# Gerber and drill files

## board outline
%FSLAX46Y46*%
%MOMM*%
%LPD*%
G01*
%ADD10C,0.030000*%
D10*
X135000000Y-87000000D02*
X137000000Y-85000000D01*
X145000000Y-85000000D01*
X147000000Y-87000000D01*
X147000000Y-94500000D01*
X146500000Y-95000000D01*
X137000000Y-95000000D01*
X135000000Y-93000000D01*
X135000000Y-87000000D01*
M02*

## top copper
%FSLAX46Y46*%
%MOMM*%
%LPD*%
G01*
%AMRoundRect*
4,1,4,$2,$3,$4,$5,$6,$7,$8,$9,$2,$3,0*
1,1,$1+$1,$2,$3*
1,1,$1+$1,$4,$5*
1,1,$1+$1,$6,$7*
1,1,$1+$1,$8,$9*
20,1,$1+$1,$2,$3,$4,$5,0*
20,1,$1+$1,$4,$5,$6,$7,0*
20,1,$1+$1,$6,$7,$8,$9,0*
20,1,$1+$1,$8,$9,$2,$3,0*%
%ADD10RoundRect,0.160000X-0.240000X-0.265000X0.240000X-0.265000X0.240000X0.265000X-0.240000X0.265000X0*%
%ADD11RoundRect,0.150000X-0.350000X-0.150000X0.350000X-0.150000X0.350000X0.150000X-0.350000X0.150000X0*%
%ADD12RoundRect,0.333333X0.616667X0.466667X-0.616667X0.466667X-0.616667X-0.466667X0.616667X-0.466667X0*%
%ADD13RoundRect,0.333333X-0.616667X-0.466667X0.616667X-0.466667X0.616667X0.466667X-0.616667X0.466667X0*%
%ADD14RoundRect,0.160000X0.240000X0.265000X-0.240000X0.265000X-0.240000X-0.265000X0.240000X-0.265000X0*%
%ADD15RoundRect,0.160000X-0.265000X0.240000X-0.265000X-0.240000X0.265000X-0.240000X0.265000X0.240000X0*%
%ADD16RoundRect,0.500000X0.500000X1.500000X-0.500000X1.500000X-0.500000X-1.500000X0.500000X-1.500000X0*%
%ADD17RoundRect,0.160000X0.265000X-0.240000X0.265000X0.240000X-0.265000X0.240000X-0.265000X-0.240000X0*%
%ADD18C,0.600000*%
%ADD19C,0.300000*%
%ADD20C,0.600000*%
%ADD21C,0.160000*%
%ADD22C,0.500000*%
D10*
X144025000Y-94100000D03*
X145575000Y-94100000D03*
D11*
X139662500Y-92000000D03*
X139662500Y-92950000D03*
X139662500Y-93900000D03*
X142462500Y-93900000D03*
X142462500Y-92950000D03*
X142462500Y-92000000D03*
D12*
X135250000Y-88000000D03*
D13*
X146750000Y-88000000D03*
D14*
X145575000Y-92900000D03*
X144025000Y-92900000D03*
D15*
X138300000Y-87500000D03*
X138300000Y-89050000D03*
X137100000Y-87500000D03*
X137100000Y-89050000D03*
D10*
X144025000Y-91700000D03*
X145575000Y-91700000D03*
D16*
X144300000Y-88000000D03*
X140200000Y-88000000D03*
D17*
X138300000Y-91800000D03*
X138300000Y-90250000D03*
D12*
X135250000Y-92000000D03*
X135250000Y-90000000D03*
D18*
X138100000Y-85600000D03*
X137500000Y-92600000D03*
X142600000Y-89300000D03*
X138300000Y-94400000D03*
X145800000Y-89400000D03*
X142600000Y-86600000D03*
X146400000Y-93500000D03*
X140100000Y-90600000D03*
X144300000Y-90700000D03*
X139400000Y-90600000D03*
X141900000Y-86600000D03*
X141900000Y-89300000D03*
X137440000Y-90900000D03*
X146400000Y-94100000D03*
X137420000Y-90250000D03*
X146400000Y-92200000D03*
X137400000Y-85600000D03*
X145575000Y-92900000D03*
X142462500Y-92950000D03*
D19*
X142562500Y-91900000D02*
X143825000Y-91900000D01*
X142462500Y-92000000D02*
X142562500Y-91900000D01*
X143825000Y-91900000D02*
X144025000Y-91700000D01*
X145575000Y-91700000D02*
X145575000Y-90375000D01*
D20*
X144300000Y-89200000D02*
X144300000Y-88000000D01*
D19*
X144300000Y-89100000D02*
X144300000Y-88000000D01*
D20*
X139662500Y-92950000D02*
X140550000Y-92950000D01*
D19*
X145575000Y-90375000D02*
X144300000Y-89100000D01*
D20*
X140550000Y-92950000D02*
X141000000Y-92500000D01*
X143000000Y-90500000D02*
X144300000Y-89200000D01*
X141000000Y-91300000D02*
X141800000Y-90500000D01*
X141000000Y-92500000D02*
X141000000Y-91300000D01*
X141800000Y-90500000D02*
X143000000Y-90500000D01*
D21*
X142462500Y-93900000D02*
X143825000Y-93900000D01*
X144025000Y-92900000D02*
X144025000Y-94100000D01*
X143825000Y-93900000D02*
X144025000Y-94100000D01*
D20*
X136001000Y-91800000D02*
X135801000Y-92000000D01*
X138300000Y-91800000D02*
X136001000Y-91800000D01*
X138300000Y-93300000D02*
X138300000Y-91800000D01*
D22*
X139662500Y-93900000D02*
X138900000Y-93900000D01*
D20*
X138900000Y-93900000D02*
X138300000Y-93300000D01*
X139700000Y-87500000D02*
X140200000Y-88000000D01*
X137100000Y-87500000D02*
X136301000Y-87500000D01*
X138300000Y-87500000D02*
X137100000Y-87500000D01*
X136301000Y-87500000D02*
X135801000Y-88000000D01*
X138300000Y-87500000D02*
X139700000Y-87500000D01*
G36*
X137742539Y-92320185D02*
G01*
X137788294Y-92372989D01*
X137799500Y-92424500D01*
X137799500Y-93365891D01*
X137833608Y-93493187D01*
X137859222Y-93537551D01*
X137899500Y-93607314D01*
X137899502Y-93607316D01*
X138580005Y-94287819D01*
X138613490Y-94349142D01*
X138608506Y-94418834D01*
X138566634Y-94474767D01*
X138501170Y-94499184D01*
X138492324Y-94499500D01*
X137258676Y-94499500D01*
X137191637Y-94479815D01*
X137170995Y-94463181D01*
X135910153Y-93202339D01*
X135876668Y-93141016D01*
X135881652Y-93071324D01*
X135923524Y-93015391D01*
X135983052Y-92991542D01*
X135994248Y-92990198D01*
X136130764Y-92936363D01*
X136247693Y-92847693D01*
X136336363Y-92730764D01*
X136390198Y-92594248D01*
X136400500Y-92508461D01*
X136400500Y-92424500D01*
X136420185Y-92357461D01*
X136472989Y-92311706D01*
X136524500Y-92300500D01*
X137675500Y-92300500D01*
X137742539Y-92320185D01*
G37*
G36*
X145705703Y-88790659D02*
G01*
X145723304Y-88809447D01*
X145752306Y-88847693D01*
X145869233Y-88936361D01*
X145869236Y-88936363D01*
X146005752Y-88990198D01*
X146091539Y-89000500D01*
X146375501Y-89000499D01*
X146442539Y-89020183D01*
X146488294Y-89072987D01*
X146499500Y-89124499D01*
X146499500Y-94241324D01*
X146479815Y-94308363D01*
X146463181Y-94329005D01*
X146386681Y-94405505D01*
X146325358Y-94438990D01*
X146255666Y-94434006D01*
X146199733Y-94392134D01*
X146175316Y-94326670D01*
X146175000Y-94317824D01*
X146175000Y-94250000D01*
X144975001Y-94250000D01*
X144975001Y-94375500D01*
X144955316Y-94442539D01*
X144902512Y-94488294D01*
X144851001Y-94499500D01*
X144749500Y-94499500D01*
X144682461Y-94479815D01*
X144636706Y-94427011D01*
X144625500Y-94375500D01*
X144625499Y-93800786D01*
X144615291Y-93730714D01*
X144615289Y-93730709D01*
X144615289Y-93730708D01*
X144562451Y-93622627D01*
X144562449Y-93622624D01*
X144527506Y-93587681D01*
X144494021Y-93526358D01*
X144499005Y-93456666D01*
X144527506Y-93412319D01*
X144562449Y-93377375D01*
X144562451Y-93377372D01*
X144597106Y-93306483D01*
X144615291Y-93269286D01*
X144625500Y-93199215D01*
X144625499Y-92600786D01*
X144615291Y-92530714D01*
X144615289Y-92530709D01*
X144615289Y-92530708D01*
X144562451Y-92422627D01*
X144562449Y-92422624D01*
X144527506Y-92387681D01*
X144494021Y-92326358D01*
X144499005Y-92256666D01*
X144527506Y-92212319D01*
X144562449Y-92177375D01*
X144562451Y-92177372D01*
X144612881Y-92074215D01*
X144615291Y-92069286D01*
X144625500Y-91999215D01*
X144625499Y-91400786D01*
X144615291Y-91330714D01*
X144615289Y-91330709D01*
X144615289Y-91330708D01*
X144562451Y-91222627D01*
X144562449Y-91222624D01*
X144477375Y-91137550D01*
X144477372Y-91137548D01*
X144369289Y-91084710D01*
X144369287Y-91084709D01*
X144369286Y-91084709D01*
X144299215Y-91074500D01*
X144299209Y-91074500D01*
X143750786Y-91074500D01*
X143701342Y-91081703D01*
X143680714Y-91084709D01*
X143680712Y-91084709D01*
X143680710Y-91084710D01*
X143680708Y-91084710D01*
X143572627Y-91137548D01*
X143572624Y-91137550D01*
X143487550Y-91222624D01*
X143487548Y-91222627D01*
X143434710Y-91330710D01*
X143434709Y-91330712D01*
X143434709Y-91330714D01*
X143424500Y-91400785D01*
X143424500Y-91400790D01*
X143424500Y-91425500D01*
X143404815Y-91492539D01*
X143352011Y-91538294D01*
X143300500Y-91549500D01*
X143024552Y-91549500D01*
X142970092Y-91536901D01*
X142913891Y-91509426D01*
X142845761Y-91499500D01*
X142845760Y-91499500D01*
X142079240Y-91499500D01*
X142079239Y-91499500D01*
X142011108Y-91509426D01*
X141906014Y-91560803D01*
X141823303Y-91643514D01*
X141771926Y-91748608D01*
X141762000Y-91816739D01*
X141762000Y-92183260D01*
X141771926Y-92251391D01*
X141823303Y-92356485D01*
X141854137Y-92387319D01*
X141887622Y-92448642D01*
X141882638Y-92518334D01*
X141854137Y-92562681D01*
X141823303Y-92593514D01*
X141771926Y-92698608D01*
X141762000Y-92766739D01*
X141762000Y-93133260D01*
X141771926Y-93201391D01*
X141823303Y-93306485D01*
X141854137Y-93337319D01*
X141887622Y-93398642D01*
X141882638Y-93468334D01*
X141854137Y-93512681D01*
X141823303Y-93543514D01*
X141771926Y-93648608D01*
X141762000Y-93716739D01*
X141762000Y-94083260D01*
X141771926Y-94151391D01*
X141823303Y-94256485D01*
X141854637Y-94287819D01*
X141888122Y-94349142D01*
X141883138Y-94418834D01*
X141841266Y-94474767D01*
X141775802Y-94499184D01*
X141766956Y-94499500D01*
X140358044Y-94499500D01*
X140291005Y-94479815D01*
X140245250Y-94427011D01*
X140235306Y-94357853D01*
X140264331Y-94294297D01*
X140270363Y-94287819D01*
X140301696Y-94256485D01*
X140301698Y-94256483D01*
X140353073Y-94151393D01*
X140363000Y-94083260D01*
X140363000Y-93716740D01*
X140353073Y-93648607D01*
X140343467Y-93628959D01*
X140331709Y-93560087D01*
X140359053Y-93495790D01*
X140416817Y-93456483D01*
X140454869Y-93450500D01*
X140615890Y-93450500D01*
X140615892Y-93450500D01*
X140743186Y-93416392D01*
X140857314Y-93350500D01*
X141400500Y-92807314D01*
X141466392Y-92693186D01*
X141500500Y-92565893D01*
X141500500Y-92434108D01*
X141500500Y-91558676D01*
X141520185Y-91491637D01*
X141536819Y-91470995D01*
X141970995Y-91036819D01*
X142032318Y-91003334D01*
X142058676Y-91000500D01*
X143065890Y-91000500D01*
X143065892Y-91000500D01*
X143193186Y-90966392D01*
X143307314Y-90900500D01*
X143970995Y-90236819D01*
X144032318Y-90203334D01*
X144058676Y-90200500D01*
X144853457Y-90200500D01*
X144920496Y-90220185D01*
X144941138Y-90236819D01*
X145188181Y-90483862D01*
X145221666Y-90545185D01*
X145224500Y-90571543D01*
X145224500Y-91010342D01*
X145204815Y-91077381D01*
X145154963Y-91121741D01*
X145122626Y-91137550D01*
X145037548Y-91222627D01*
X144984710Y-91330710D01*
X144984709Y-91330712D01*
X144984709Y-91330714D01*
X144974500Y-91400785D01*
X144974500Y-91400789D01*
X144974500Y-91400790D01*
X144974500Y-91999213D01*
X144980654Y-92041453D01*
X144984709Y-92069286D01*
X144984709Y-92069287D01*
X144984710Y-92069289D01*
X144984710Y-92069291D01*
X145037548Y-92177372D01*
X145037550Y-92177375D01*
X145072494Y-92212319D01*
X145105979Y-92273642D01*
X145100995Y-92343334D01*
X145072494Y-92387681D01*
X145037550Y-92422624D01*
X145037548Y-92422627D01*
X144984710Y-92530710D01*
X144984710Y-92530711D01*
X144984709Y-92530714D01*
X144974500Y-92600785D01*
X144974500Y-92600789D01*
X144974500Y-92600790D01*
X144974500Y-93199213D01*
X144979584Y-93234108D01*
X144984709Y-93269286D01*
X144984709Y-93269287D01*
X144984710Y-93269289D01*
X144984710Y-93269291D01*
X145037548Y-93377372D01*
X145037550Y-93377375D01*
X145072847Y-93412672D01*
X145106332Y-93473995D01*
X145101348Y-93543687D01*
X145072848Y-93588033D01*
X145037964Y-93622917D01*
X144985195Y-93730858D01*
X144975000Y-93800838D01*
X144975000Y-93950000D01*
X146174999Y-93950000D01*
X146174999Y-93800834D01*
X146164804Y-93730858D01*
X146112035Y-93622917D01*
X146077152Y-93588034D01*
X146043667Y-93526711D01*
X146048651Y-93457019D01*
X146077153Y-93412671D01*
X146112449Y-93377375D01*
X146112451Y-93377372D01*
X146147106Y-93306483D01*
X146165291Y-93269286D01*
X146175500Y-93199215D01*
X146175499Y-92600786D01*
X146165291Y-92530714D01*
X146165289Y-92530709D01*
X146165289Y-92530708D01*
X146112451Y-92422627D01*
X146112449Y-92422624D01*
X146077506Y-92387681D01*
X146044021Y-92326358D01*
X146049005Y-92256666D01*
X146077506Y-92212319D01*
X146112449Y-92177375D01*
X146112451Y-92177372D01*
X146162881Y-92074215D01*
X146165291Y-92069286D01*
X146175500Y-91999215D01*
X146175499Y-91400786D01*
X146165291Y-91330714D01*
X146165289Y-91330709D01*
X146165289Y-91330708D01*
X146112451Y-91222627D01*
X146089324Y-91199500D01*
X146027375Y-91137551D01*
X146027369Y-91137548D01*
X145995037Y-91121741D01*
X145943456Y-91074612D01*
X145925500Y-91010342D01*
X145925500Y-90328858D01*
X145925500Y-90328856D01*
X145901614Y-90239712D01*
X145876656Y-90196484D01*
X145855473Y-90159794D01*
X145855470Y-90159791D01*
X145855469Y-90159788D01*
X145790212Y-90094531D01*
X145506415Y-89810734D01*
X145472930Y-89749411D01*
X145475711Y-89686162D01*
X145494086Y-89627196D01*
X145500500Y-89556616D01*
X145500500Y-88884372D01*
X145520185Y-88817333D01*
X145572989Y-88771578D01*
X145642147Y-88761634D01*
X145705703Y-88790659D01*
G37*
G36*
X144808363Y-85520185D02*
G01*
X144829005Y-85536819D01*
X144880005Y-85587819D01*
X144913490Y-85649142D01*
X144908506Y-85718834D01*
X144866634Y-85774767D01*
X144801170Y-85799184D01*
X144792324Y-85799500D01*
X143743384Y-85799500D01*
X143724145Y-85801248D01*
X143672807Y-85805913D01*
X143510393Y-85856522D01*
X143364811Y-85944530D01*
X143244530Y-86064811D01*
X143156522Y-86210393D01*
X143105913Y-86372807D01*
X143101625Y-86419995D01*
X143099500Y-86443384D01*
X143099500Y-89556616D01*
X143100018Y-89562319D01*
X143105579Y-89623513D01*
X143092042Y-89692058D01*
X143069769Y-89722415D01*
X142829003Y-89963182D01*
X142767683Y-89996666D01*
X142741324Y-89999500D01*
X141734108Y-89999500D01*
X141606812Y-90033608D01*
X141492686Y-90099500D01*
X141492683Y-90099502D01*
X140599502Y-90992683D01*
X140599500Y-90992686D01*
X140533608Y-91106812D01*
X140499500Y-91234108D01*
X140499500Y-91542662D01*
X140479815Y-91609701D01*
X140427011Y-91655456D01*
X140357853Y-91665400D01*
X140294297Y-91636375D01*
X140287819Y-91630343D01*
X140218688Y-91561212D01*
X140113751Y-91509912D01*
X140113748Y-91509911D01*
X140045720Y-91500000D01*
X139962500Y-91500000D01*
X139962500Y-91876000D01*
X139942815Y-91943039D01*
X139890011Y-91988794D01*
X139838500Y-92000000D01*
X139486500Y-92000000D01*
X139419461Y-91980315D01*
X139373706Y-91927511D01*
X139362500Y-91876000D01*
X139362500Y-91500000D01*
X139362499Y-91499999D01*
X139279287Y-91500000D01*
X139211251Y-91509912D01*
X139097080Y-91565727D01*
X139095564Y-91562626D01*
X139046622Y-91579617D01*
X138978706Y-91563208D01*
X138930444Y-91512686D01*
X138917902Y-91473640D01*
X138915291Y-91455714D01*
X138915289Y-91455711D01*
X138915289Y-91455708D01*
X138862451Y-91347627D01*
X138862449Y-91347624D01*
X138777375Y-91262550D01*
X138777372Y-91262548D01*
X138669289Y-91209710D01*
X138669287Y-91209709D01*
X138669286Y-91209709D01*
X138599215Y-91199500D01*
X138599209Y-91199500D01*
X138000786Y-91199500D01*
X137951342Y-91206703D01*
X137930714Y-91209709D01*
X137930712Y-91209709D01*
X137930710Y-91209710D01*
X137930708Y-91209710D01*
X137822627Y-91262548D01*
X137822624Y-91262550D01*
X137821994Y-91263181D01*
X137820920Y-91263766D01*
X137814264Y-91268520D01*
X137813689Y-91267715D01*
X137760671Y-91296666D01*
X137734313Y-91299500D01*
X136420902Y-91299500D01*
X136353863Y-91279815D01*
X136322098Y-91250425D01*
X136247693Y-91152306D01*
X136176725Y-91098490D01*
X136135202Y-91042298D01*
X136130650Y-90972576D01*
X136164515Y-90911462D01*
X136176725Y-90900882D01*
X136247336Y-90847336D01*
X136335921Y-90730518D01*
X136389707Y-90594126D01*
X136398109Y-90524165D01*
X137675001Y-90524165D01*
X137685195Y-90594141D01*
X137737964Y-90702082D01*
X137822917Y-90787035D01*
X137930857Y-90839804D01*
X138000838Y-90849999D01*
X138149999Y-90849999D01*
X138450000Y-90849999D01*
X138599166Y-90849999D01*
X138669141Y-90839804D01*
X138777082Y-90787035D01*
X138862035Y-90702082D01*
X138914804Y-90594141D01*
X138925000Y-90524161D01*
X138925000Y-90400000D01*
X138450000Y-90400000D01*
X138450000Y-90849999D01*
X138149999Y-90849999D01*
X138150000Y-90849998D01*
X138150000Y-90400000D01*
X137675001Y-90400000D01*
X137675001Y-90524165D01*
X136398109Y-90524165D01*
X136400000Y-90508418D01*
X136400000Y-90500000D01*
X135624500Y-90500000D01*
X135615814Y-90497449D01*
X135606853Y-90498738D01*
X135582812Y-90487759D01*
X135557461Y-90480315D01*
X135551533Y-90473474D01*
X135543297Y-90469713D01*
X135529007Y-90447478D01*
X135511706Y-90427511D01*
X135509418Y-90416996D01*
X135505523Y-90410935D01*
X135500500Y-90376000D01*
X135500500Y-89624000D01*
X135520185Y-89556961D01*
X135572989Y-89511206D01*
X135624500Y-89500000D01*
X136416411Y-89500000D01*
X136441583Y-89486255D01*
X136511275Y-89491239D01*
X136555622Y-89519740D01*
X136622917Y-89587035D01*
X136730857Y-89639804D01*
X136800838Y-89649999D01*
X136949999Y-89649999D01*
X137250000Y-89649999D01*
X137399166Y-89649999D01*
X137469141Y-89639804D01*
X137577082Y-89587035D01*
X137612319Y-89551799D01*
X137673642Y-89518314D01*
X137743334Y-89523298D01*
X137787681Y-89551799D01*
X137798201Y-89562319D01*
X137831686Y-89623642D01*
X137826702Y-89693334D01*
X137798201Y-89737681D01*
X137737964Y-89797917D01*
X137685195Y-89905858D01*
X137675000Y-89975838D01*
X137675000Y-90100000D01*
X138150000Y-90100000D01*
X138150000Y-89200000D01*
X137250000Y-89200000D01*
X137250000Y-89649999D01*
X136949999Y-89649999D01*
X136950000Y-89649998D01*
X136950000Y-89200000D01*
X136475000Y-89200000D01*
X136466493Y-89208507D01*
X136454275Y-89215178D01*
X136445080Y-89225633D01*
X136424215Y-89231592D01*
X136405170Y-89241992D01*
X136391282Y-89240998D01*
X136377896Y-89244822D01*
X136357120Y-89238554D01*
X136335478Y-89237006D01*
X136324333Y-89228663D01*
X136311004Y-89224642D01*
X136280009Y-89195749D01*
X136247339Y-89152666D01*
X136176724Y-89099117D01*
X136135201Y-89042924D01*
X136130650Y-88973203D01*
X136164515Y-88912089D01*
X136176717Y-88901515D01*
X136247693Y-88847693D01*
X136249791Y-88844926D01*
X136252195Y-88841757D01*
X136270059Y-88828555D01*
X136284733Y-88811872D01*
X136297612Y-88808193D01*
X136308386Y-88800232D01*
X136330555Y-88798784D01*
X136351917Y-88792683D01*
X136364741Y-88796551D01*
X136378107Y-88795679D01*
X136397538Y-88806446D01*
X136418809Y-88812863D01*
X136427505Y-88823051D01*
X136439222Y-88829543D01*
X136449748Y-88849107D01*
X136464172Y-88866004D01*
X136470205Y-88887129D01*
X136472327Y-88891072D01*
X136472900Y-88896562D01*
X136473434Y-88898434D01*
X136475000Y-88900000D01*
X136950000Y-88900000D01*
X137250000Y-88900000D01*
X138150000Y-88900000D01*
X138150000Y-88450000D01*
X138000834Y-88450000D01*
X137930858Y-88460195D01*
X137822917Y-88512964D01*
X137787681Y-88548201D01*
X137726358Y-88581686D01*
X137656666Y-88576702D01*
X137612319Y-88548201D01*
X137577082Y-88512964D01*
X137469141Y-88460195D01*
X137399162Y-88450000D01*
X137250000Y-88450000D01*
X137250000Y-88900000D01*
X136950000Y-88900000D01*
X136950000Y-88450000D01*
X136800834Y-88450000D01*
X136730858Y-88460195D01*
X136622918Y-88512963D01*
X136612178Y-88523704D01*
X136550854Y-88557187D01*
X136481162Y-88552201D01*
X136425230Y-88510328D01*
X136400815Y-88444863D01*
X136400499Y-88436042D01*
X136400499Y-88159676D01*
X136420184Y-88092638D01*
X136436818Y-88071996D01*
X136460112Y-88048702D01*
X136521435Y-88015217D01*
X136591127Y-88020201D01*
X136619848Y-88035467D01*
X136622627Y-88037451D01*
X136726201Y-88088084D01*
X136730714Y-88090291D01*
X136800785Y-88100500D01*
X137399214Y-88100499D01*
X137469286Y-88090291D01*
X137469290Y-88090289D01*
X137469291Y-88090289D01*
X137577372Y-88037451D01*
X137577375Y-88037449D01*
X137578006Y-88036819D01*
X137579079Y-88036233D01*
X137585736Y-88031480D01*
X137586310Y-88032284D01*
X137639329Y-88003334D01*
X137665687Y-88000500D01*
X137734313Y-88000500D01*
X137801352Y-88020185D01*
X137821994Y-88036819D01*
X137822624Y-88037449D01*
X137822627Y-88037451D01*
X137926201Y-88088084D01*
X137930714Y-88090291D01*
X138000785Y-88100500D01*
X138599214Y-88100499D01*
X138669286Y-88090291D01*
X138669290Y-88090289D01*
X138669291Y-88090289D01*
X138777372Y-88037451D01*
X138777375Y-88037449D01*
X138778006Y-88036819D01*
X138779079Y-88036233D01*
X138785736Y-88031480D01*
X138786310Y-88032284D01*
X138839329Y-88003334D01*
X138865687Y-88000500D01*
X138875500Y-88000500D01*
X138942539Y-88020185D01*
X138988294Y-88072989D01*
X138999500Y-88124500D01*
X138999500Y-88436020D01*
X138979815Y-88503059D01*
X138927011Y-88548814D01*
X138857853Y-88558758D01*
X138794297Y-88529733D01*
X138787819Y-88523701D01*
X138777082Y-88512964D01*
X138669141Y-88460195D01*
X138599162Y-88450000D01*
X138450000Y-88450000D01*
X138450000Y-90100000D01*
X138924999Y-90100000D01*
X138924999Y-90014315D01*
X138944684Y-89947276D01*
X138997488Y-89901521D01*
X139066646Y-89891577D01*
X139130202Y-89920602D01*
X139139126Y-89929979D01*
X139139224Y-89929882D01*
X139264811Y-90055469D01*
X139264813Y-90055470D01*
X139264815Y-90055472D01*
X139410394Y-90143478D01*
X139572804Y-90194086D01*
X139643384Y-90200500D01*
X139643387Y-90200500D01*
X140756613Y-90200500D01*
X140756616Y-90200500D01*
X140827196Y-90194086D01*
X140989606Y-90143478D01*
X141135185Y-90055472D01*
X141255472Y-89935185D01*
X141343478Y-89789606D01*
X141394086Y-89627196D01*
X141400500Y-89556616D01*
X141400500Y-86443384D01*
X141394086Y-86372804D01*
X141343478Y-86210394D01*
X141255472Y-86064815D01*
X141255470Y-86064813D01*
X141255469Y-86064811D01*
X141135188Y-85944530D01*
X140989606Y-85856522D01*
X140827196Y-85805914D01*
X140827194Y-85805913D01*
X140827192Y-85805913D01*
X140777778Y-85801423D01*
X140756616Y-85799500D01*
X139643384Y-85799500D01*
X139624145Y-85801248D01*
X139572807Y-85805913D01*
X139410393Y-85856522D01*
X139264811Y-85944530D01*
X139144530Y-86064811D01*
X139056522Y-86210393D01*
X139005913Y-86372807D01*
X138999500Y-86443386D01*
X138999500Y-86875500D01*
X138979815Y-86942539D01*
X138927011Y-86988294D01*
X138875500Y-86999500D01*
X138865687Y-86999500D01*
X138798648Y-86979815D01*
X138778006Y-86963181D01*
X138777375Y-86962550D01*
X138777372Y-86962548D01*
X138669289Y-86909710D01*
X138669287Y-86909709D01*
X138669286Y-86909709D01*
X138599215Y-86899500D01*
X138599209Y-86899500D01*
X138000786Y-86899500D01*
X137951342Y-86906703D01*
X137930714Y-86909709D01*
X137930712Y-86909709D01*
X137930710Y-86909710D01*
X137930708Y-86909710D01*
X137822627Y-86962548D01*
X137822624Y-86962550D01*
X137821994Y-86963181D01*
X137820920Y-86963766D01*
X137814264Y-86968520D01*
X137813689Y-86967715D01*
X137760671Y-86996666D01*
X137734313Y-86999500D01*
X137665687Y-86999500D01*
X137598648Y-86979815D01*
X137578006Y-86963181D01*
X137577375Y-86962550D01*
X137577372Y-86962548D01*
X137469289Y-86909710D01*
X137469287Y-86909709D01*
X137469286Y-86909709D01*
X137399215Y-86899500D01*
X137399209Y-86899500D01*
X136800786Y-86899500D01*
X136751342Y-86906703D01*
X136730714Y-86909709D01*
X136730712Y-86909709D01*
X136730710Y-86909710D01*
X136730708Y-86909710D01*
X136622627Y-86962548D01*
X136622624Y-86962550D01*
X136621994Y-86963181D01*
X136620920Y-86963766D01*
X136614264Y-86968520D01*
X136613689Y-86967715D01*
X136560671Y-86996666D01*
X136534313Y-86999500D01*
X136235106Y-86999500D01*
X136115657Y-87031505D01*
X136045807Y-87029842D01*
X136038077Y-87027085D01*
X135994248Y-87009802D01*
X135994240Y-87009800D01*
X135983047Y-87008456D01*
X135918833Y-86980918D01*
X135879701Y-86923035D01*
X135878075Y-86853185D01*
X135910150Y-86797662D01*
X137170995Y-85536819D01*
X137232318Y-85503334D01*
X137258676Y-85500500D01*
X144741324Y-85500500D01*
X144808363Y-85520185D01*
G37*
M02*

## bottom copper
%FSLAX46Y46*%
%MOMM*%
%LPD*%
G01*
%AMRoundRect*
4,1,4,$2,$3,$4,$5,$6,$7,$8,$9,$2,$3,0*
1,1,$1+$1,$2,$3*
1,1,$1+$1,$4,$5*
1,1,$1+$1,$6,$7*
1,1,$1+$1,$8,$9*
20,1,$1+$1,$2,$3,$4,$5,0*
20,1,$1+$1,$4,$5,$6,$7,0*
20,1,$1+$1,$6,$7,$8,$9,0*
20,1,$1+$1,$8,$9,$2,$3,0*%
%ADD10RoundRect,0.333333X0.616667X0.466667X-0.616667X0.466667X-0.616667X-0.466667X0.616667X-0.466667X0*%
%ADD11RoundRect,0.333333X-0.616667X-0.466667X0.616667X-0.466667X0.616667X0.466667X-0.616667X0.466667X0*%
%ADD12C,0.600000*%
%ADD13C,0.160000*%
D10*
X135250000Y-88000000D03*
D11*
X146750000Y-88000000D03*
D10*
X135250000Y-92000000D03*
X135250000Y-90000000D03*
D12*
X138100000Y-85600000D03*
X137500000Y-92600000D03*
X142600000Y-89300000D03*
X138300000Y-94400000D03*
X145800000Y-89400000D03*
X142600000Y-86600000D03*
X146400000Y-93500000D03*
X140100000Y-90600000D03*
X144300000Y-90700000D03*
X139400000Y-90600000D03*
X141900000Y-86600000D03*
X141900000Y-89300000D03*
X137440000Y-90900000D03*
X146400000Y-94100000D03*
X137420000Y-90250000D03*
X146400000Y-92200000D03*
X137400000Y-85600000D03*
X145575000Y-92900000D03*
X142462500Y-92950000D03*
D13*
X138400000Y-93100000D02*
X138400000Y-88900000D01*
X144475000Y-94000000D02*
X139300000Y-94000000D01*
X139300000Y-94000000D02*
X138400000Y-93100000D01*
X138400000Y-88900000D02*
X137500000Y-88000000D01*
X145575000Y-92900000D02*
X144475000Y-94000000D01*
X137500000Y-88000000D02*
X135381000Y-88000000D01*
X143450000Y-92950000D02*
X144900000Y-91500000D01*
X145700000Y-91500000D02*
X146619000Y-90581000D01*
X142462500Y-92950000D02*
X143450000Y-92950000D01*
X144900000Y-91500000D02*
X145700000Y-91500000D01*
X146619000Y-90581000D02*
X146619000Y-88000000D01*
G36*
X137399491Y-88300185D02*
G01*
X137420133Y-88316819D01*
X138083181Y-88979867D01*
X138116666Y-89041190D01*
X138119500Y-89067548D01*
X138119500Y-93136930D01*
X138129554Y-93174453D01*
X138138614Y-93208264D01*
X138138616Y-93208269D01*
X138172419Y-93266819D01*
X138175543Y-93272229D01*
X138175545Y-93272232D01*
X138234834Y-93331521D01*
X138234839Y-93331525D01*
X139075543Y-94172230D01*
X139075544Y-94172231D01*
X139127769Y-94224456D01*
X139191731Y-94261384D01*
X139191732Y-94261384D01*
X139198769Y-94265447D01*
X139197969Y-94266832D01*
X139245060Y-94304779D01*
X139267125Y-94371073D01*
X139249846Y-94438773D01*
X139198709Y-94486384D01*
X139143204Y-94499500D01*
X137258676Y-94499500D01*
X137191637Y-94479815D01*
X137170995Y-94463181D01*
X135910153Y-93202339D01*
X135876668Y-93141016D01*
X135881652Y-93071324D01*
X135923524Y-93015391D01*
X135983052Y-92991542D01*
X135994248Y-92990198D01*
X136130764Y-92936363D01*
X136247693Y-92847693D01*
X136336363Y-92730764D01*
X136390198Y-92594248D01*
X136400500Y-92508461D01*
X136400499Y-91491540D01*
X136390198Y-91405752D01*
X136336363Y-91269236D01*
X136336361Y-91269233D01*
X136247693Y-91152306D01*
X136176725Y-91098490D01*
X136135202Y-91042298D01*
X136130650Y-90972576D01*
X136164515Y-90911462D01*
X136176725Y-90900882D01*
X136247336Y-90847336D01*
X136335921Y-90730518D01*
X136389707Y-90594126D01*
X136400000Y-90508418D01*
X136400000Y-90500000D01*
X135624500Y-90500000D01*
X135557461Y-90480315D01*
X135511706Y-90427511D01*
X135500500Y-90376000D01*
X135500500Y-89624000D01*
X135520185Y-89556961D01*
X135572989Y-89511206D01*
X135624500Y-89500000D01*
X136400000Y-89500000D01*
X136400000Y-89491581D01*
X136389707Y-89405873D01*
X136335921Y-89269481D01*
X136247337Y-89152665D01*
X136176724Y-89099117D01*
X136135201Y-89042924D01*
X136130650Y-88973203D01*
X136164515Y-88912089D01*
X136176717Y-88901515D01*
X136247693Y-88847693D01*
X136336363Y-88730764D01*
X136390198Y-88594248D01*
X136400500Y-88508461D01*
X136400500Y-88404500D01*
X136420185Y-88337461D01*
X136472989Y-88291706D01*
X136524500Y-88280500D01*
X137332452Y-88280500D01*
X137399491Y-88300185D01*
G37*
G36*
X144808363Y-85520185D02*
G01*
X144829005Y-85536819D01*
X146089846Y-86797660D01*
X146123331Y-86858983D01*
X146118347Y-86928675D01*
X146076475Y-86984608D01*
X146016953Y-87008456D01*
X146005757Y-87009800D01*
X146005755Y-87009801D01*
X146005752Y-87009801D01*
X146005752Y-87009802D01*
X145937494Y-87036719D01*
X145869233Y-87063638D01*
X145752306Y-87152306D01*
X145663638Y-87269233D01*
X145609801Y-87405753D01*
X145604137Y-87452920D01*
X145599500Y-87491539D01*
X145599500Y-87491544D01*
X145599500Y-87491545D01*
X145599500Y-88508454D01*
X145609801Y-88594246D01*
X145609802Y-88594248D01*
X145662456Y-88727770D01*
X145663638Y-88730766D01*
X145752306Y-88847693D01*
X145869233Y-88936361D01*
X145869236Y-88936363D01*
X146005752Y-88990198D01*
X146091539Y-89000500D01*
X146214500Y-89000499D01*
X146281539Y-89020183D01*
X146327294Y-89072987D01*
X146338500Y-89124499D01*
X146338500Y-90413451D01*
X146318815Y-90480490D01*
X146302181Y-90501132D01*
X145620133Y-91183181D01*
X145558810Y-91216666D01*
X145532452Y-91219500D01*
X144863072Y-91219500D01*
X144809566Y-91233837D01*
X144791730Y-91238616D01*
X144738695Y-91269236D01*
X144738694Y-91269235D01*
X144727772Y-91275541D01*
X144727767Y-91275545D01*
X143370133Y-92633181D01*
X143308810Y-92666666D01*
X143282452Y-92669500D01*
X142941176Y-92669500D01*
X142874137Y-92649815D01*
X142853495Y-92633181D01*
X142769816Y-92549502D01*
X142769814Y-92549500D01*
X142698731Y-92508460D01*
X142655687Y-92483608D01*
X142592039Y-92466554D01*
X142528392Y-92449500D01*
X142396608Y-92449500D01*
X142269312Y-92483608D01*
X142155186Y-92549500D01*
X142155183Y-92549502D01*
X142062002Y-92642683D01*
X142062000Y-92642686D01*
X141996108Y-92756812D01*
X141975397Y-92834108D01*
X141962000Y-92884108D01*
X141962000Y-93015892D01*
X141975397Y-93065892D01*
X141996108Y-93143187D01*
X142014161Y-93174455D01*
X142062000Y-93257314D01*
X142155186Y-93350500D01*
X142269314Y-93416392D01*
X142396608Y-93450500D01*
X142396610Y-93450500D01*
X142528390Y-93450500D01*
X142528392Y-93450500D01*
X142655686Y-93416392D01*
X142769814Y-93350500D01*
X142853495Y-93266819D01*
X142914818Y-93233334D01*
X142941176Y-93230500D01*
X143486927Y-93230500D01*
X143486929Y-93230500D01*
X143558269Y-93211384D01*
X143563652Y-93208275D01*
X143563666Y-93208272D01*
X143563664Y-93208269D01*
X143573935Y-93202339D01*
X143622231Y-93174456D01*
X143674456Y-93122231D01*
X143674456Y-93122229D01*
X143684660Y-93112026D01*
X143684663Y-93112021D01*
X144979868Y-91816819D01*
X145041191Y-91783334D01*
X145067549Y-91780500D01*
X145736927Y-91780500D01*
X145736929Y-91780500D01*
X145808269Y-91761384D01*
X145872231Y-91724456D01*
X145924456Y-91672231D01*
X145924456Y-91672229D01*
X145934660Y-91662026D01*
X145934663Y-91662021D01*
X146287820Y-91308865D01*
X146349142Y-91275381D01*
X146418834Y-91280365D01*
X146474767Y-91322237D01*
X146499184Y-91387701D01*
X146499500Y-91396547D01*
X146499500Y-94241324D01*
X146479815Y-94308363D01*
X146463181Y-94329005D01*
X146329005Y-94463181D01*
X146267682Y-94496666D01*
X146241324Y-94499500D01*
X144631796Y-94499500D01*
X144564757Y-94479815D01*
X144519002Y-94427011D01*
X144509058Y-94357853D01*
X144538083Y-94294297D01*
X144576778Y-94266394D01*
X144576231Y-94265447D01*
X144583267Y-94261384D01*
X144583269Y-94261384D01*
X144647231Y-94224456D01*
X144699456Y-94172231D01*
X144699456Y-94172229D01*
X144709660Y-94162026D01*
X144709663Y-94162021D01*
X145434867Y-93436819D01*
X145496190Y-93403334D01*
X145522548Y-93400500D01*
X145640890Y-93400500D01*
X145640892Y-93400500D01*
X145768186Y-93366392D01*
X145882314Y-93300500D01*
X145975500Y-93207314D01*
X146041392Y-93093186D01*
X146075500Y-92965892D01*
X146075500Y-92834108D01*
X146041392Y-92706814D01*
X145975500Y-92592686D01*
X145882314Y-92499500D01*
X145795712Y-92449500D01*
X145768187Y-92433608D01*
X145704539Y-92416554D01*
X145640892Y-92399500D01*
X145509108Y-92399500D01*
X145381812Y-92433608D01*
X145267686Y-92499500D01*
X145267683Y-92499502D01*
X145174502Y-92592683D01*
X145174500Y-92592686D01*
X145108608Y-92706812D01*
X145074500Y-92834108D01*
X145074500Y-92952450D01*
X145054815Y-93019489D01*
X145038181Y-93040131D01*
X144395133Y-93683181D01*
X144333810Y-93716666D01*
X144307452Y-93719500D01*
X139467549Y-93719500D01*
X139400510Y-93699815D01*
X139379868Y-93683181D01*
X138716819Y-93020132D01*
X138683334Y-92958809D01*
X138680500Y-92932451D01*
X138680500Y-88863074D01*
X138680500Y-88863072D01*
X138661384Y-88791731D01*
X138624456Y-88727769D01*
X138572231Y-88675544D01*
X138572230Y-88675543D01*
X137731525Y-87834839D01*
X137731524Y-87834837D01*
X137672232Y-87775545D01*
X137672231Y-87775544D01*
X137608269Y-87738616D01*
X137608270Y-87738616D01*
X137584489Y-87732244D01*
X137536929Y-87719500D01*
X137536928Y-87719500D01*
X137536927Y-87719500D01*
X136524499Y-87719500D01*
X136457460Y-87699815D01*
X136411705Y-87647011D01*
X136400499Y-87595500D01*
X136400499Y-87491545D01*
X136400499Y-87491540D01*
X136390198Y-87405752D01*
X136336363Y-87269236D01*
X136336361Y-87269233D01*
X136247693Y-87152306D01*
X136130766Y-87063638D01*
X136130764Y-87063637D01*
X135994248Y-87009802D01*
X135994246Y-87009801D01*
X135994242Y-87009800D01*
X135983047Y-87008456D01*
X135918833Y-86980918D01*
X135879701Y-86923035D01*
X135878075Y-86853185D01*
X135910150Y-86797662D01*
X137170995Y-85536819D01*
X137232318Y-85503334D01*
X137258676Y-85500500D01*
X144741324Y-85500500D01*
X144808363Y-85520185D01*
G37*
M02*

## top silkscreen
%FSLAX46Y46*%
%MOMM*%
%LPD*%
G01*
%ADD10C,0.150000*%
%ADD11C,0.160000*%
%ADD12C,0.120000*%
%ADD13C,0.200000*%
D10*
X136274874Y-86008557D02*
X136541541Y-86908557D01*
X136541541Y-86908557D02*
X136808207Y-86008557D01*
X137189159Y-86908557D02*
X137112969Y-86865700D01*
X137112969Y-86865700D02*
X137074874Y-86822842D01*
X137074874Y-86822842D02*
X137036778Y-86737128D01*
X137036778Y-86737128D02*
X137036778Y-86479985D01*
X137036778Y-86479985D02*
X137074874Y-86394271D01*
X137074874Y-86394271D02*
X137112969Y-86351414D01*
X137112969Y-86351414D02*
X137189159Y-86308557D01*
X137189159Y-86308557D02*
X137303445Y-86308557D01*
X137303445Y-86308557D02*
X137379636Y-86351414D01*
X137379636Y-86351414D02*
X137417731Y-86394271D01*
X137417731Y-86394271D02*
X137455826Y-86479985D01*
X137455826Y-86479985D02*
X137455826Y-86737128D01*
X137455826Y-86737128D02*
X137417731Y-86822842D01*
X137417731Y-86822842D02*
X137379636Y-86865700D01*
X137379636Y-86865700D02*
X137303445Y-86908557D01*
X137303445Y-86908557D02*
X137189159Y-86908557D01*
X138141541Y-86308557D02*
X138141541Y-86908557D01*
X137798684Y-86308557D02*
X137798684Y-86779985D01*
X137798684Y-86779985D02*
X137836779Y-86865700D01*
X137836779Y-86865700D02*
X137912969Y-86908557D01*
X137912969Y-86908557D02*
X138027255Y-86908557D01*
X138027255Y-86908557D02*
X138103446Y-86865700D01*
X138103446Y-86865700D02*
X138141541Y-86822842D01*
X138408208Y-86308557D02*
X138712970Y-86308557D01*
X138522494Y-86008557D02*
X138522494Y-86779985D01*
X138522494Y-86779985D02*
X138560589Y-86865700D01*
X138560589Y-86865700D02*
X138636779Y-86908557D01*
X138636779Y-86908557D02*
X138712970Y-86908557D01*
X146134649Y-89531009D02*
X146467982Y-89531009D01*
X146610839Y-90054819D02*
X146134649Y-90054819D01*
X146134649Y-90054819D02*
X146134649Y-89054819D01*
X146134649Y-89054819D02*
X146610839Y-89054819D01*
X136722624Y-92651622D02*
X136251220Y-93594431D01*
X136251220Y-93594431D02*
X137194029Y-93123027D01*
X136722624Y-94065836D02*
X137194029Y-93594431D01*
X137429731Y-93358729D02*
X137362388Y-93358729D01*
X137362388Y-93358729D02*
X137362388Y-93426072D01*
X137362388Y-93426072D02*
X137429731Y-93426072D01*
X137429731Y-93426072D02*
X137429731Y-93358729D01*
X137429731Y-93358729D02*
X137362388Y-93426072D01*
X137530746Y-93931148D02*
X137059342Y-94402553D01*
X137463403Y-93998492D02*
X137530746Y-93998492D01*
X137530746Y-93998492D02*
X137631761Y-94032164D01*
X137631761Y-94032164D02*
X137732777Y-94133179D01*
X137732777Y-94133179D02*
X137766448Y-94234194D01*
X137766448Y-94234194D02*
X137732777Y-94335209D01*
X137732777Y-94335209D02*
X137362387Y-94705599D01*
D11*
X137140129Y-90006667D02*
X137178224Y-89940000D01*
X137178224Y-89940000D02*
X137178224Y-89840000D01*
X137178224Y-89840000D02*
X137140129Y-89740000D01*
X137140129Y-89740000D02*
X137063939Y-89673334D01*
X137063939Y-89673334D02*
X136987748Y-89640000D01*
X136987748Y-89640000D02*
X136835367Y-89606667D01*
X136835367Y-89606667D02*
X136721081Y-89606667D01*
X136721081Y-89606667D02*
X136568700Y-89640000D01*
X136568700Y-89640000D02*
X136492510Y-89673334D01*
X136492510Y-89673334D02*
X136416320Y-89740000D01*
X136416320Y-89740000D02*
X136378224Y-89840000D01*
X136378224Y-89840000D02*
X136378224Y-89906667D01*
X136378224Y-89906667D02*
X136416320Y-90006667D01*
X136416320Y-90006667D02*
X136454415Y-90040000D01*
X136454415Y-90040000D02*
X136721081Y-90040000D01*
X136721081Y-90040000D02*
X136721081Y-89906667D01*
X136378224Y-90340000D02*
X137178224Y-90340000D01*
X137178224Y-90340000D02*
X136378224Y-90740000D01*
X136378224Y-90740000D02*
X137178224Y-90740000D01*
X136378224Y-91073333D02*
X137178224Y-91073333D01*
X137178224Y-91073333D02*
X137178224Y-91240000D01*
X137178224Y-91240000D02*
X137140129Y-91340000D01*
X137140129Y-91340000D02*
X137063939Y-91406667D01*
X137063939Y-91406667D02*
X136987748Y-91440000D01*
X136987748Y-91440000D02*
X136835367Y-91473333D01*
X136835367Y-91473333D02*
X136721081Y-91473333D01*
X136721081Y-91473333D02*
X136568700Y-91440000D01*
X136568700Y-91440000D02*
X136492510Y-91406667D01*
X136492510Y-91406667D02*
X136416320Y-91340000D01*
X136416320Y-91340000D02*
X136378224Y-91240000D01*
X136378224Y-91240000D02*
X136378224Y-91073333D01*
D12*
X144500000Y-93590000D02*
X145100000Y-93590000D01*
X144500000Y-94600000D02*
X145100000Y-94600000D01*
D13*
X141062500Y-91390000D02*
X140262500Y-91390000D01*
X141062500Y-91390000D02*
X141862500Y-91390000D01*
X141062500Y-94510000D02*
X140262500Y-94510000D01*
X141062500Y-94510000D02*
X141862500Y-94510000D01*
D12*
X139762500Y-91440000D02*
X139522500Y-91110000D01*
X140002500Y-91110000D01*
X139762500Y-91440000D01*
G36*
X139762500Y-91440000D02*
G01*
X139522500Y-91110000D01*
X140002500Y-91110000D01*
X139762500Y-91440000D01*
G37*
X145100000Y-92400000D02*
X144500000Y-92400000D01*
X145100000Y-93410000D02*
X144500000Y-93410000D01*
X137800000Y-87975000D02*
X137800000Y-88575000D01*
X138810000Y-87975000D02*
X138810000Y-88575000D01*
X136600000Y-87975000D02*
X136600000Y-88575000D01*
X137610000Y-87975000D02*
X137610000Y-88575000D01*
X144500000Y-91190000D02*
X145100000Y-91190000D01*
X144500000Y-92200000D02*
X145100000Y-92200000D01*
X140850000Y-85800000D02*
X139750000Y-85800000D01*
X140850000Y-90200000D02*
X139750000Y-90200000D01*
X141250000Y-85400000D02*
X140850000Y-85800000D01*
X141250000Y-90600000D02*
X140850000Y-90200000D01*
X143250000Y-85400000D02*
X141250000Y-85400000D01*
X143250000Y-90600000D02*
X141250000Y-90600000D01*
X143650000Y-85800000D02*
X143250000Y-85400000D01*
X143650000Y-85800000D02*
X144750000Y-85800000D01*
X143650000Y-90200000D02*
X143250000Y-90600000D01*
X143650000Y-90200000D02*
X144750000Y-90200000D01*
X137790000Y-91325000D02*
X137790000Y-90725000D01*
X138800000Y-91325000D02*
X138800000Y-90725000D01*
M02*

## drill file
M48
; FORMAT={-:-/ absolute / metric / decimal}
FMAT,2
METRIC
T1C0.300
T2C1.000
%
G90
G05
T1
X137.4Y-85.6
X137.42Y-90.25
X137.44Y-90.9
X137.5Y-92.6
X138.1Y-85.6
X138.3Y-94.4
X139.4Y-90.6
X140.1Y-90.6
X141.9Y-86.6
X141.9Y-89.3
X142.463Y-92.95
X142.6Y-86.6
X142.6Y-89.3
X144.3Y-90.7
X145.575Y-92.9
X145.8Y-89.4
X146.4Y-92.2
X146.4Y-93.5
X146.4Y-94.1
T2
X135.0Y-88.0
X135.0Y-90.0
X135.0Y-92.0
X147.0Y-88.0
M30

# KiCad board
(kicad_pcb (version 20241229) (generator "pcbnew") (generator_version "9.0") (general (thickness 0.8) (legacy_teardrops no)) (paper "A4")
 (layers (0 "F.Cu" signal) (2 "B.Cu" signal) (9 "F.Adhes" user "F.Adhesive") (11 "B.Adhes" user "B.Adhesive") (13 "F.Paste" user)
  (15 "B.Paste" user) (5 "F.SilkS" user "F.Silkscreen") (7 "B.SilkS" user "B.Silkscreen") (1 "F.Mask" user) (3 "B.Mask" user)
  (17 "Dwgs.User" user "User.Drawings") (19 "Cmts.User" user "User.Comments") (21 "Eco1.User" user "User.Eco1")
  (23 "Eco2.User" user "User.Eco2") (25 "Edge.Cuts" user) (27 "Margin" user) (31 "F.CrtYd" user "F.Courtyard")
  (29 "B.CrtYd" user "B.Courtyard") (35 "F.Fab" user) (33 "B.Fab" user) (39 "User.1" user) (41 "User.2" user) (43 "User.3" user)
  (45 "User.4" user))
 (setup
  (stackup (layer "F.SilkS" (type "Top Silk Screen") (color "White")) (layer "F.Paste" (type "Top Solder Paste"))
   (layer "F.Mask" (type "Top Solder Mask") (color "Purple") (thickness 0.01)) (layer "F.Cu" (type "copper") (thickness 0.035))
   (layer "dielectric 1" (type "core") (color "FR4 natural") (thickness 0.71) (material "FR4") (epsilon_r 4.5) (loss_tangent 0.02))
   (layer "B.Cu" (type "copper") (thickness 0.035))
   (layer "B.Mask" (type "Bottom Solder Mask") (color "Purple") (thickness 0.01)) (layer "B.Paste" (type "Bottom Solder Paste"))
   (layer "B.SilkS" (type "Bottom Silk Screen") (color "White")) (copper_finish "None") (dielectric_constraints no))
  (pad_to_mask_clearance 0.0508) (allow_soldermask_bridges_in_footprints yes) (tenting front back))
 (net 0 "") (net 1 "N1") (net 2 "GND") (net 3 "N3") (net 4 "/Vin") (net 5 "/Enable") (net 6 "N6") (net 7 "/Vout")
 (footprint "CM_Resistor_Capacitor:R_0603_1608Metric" (layer "F.Cu") (at 144.8 94.1)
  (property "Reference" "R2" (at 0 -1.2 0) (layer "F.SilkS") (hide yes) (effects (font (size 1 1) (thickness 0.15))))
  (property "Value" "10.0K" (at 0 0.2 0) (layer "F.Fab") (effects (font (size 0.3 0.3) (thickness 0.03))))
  (fp_line (start -0.3 -0.51) (end 0.3 -0.51) (stroke (width 0.12) (type solid)) (layer "F.SilkS"))
  (fp_line (start -0.3 0.5) (end 0.3 0.5) (stroke (width 0.12) (type solid)) (layer "F.SilkS"))
  (pad "1" smd roundrect (at -0.775 0) (size 0.8 0.85) (layers "F.Cu" "F.Mask" "F.Paste") (roundrect_rratio 0.2) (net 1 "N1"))
  (pad "2" smd roundrect (at 0.775 0) (size 0.8 0.85) (layers "F.Cu" "F.Mask" "F.Paste") (roundrect_rratio 0.2) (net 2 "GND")))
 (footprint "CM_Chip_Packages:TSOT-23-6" (layer "F.Cu") (at 141.0625 92.95)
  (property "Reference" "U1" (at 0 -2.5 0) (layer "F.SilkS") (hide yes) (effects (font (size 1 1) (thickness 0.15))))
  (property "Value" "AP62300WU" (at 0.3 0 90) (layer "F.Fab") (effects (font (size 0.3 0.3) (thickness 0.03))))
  (fp_line (start 0 -1.56) (end -0.8 -1.56) (stroke (width 0.2) (type solid)) (layer "F.SilkS"))
  (fp_line (start 0 -1.56) (end 0.8 -1.56) (stroke (width 0.2) (type solid)) (layer "F.SilkS"))
  (fp_line (start 0 1.56) (end -0.8 1.56) (stroke (width 0.2) (type solid)) (layer "F.SilkS"))
  (fp_line (start 0 1.56) (end 0.8 1.56) (stroke (width 0.2) (type solid)) (layer "F.SilkS"))
  (fp_poly (pts (xy -1.3 -1.51) (xy -1.54 -1.84) (xy -1.06 -1.84)) (stroke (width 0.12) (type solid)) (fill yes) (layer "F.SilkS"))
  (pad "1" smd roundrect (at -1.4 -0.95) (size 1 0.6) (layers "F.Cu" "F.Mask" "F.Paste") (roundrect_rratio 0.25) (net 2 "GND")
   (thermal_bridge_width 0.6))
  (pad "2" smd roundrect (at -1.4 0) (size 1 0.6) (layers "F.Cu" "F.Mask" "F.Paste") (roundrect_rratio 0.25) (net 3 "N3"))
  (pad "3" smd roundrect (at -1.4 0.95) (size 1 0.6) (layers "F.Cu" "F.Mask" "F.Paste") (roundrect_rratio 0.25) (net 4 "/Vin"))
  (pad "4" smd roundrect (at 1.4 0.95) (size 1 0.6) (layers "F.Cu" "F.Mask" "F.Paste") (roundrect_rratio 0.25) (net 1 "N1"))
  (pad "5" smd roundrect (at 1.4 0) (size 1 0.6) (layers "F.Cu" "F.Mask" "F.Paste") (roundrect_rratio 0.25) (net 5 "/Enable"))
  (pad "6" smd roundrect (at 1.4 -0.95) (size 1 0.6) (layers "F.Cu" "F.Mask" "F.Paste") (roundrect_rratio 0.25) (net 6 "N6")))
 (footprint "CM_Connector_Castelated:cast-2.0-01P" (layer "F.Cu") (at 135 88 180)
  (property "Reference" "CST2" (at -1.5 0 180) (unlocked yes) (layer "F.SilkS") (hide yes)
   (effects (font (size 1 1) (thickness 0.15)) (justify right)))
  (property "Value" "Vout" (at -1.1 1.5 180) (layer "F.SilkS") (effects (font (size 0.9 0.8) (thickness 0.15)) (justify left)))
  (pad "1" thru_hole roundrect (at 0 0 180) (size 1.9 1.6) (drill 1 (offset -0.25 0)) (layers "*.Cu" "*.Mask") (remove_unused_layers no)
   (roundrect_rratio 0.2083333333) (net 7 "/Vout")))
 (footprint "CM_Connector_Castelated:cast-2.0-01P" (layer "F.Cu") (at 147 88)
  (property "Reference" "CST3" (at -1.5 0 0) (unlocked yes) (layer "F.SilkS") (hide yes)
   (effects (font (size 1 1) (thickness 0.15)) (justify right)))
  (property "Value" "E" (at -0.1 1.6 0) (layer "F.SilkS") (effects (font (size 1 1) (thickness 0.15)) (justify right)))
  (pad "1" thru_hole roundrect (at 0 0) (size 1.9 1.6) (drill 1 (offset -0.25 0)) (layers "*.Cu" "*.Mask") (remove_unused_layers no)
   (roundrect_rratio 0.2083333333) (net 5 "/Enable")))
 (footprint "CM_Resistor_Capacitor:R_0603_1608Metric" (layer "F.Cu") (at 144.8 92.9 180)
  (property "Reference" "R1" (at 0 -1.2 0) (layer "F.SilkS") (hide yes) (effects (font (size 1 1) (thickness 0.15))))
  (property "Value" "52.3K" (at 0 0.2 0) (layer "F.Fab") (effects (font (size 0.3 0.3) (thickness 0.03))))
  (fp_line (start -0.3 0.5) (end 0.3 0.5) (stroke (width 0.12) (type solid)) (layer "F.SilkS"))
  (fp_line (start -0.3 -0.51) (end 0.3 -0.51) (stroke (width 0.12) (type solid)) (layer "F.SilkS"))
  (pad "1" smd roundrect (at -0.775 0 180) (size 0.8 0.85) (layers "F.Cu" "F.Mask" "F.Paste") (roundrect_rratio 0.2) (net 7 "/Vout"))
  (pad "2" smd roundrect (at 0.775 0 180) (size 0.8 0.85) (layers "F.Cu" "F.Mask" "F.Paste") (roundrect_rratio 0.2) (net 1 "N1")))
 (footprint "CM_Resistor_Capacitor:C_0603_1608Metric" (layer "F.Cu") (at 138.3 88.275 -90)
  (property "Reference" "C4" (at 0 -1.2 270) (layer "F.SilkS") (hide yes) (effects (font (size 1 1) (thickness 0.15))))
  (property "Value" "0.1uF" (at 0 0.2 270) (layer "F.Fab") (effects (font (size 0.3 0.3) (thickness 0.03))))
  (fp_line (start -0.3 0.5) (end 0.3 0.5) (stroke (width 0.12) (type solid)) (layer "F.SilkS"))
  (fp_line (start -0.3 -0.51) (end 0.3 -0.51) (stroke (width 0.12) (type solid)) (layer "F.SilkS"))
  (pad "1" smd roundrect (at -0.775 0 270) (size 0.8 0.85) (layers "F.Cu" "F.Mask" "F.Paste") (roundrect_rratio 0.2) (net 7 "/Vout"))
  (pad "2" smd roundrect (at 0.775 0 270) (size 0.8 0.85) (layers "F.Cu" "F.Mask" "F.Paste") (roundrect_rratio 0.2) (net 2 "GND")))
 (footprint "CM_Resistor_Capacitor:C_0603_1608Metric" (layer "F.Cu") (at 137.1 88.275 -90)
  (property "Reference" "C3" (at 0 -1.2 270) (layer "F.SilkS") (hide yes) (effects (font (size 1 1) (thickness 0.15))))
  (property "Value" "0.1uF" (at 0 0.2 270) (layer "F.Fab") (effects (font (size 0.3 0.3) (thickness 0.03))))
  (fp_line (start -0.3 0.5) (end 0.3 0.5) (stroke (width 0.12) (type solid)) (layer "F.SilkS"))
  (fp_line (start -0.3 -0.51) (end 0.3 -0.51) (stroke (width 0.12) (type solid)) (layer "F.SilkS"))
  (pad "1" smd roundrect (at -0.775 0 270) (size 0.8 0.85) (layers "F.Cu" "F.Mask" "F.Paste") (roundrect_rratio 0.2) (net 7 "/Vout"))
  (pad "2" smd roundrect (at 0.775 0 270) (size 0.8 0.85) (layers "F.Cu" "F.Mask" "F.Paste") (roundrect_rratio 0.2) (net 2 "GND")))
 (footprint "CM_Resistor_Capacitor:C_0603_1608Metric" (layer "F.Cu") (at 144.8 91.7)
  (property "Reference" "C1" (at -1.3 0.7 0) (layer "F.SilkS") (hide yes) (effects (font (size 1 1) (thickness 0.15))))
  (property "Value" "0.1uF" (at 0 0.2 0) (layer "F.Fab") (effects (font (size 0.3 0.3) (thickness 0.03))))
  (fp_line (start -0.3 -0.51) (end 0.3 -0.51) (stroke (width 0.12) (type solid)) (layer "F.SilkS"))
  (fp_line (start -0.3 0.5) (end 0.3 0.5) (stroke (width 0.12) (type solid)) (layer "F.SilkS"))
  (pad "1" smd roundrect (at -0.775 0) (size 0.8 0.85) (layers "F.Cu" "F.Mask" "F.Paste") (roundrect_rratio 0.2) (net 6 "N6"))
  (pad "2" smd roundrect (at 0.775 0) (size 0.8 0.85) (layers "F.Cu" "F.Mask" "F.Paste") (roundrect_rratio 0.2) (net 3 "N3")))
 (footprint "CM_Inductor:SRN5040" (layer "F.Cu") (at 142.25 88 180)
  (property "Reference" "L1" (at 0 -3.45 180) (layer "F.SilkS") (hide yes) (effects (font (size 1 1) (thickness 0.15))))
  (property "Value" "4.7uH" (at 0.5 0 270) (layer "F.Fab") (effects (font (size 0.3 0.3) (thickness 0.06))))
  (fp_line (start 1.4 2.2) (end 2.5 2.2) (stroke (width 0.12) (type default)) (layer "F.SilkS"))
  (fp_line (start 1.4 -2.2) (end 2.5 -2.2) (stroke (width 0.12) (type default)) (layer "F.SilkS"))
  (fp_line (start 1 2.6) (end 1.4 2.2) (stroke (width 0.12) (type default)) (layer "F.SilkS"))
  (fp_line (start 1 -2.6) (end 1.4 -2.2) (stroke (width 0.12) (type default)) (layer "F.SilkS"))
  (fp_line (start -1 2.6) (end 1 2.6) (stroke (width 0.12) (type default)) (layer "F.SilkS"))
  (fp_line (start -1 -2.6) (end 1 -2.6) (stroke (width 0.12) (type default)) (layer "F.SilkS"))
  (fp_line (start -1.4 2.2) (end -1 2.6) (stroke (width 0.12) (type default)) (layer "F.SilkS"))
  (fp_line (start -1.4 2.2) (end -2.5 2.2) (stroke (width 0.12) (type default)) (layer "F.SilkS"))
  (fp_line (start -1.4 -2.2) (end -1 -2.6) (stroke (width 0.12) (type default)) (layer "F.SilkS"))
  (fp_line (start -1.4 -2.2) (end -2.5 -2.2) (stroke (width 0.12) (type default)) (layer "F.SilkS"))
  (pad "1" smd roundrect (at -2.05 0 180) (size 2 4) (layers "F.Cu" "F.Mask" "F.Paste") (roundrect_rratio 0.25) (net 3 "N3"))
  (pad "2" smd roundrect (at 2.05 0 180) (size 2 4) (layers "F.Cu" "F.Mask" "F.Paste") (roundrect_rratio 0.25) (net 7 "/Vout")))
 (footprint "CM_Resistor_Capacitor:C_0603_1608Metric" (layer "F.Cu") (at 138.3 91.025 90)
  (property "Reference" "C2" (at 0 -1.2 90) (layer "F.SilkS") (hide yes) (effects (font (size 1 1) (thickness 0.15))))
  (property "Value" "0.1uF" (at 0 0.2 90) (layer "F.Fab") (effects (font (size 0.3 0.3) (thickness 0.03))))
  (fp_line (start -0.3 -0.51) (end 0.3 -0.51) (stroke (width 0.12) (type solid)) (layer "F.SilkS"))
  (fp_line (start -0.3 0.5) (end 0.3 0.5) (stroke (width 0.12) (type solid)) (layer "F.SilkS"))
  (pad "1" smd roundrect (at -0.775 0 90) (size 0.8 0.85) (layers "F.Cu" "F.Mask" "F.Paste") (roundrect_rratio 0.2) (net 4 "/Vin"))
  (pad "2" smd roundrect (at 0.775 0 90) (size 0.8 0.85) (layers "F.Cu" "F.Mask" "F.Paste") (roundrect_rratio 0.2) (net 2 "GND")))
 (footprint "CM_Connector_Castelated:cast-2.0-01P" (layer "F.Cu") (at 135 92 180)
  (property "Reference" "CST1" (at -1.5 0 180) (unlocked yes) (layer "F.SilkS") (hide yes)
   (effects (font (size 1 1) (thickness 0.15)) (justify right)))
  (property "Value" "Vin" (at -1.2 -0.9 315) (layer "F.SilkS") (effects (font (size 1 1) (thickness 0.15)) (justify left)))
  (pad "1" thru_hole roundrect (at 0 0 180) (size 1.9 1.6) (drill 1 (offset -0.25 0)) (layers "*.Cu" "*.Mask") (remove_unused_layers no)
   (roundrect_rratio 0.2083333333) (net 4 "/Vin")))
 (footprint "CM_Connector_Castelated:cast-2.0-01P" (layer "F.Cu") (at 135 90 180)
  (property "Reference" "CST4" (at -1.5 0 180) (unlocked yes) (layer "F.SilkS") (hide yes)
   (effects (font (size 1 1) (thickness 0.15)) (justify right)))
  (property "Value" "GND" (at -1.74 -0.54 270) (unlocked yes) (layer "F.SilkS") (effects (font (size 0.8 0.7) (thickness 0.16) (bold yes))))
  (pad "1" thru_hole roundrect (at 0 0 180) (size 1.9 1.6) (drill 1 (offset -0.25 0)) (layers "*.Cu" "*.Mask") (remove_unused_layers no)
   (roundrect_rratio 0.2083333333) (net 2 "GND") (thermal_bridge_width 1)))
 (gr_poly
  (pts (xy 135 87) (xy 137 85) (xy 145 85) (xy 147 87) (xy 147 94.5) (xy 146.5 95) (xy 137 95) (xy 135 93))
  (stroke (width 0.03) (type solid)) (fill no) (layer "Edge.Cuts"))
 (segment (start 142.5625 91.9) (end 143.825 91.9) (width 0.3) (layer "F.Cu") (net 6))
 (segment (start 142.4625 92) (end 142.5625 91.9) (width 0.3) (layer "F.Cu") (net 6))
 (segment (start 143.825 91.9) (end 144.025 91.7) (width 0.3) (layer "F.Cu") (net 6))
 (segment (start 145.575 91.7) (end 145.575 90.375) (width 0.3) (layer "F.Cu") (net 3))
 (segment (start 144.3 89.2) (end 144.3 88) (width 0.6) (layer "F.Cu") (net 3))
 (segment (start 144.3 89.1) (end 144.3 88) (width 0.3) (layer "F.Cu") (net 3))
 (segment (start 139.6625 92.95) (end 140.55 92.95) (width 0.6) (layer "F.Cu") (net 3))
 (segment (start 145.575 90.375) (end 144.3 89.1) (width 0.3) (layer "F.Cu") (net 3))
 (segment (start 140.55 92.95) (end 141 92.5) (width 0.6) (layer "F.Cu") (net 3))
 (segment (start 143 90.5) (end 144.3 89.2) (width 0.6) (layer "F.Cu") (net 3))
 (segment (start 141 91.3) (end 141.8 90.5) (width 0.6) (layer "F.Cu") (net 3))
 (segment (start 141 92.5) (end 141 91.3) (width 0.6) (layer "F.Cu") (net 3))
 (segment (start 141.8 90.5) (end 143 90.5) (width 0.6) (layer "F.Cu") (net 3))
 (via (at 138.1 85.6) (size 0.6) (drill 0.3) (layers "F.Cu" "B.Cu") (free yes) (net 2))
 (via (at 137.5 92.6) (size 0.6) (drill 0.3) (layers "F.Cu" "B.Cu") (free yes) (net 2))
 (via (at 142.6 89.3) (size 0.6) (drill 0.3) (layers "F.Cu" "B.Cu") (free yes) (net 2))
 (via (at 138.3 94.4) (size 0.6) (drill 0.3) (layers "F.Cu" "B.Cu") (free yes) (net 2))
 (via (at 145.8 89.4) (size 0.6) (drill 0.3) (layers "F.Cu" "B.Cu") (free yes) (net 2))
 (via (at 142.6 86.6) (size 0.6) (drill 0.3) (layers "F.Cu" "B.Cu") (free yes) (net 2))
 (via (at 146.4 93.5) (size 0.6) (drill 0.3) (layers "F.Cu" "B.Cu") (free yes) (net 2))
 (via (at 140.1 90.6) (size 0.6) (drill 0.3) (layers "F.Cu" "B.Cu") (free yes) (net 2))
 (via (at 144.3 90.7) (size 0.6) (drill 0.3) (layers "F.Cu" "B.Cu") (free yes) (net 2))
 (via (at 139.4 90.6) (size 0.6) (drill 0.3) (layers "F.Cu" "B.Cu") (free yes) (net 2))
 (via (at 141.9 86.6) (size 0.6) (drill 0.3) (layers "F.Cu" "B.Cu") (free yes) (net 2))
 (via (at 141.9 89.3) (size 0.6) (drill 0.3) (layers "F.Cu" "B.Cu") (free yes) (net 2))
 (via (at 137.44 90.9) (size 0.6) (drill 0.3) (layers "F.Cu" "B.Cu") (free yes) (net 2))
 (via (at 146.4 94.1) (size 0.6) (drill 0.3) (layers "F.Cu" "B.Cu") (free yes) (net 2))
 (via (at 137.42 90.25) (size 0.6) (drill 0.3) (layers "F.Cu" "B.Cu") (free yes) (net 2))
 (via (at 146.4 92.2) (size 0.6) (drill 0.3) (layers "F.Cu" "B.Cu") (free yes) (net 2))
 (via (at 137.4 85.6) (size 0.6) (drill 0.3) (layers "F.Cu" "B.Cu") (free yes) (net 2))
 (segment (start 142.4625 93.9) (end 143.825 93.9) (width 0.16) (layer "F.Cu") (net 1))
 (segment (start 144.025 92.9) (end 144.025 94.1) (width 0.16) (layer "F.Cu") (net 1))
 (segment (start 143.825 93.9) (end 144.025 94.1) (width 0.16) (layer "F.Cu") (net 1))
 (segment (start 136.001 91.8) (end 135.801 92) (width 0.6) (layer "F.Cu") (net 4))
 (segment (start 138.3 91.8) (end 136.001 91.8) (width 0.6) (layer "F.Cu") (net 4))
 (segment (start 138.3 93.3) (end 138.3 91.8) (width 0.6) (layer "F.Cu") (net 4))
 (segment (start 139.6625 93.9) (end 138.9 93.9) (width 0.5) (layer "F.Cu") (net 4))
 (segment (start 138.9 93.9) (end 138.3 93.3) (width 0.6) (layer "F.Cu") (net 4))
 (segment (start 139.7 87.5) (end 140.2 88) (width 0.6) (layer "F.Cu") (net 7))
 (segment (start 137.1 87.5) (end 136.301 87.5) (width 0.6) (layer "F.Cu") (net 7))
 (segment (start 138.3 87.5) (end 137.1 87.5) (width 0.6) (layer "F.Cu") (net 7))
 (segment (start 136.301 87.5) (end 135.801 88) (width 0.6) (layer "F.Cu") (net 7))
 (segment (start 138.3 87.5) (end 139.7 87.5) (width 0.6) (layer "F.Cu") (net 7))
 (via (at 145.575 92.9) (size 0.6) (drill 0.3) (layers "F.Cu" "B.Cu") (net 7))
 (segment (start 138.4 93.1) (end 138.4 88.9) (width 0.16) (layer "B.Cu") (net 7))
 (segment (start 144.475 94) (end 139.3 94) (width 0.16) (layer "B.Cu") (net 7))
 (segment (start 139.3 94) (end 138.4 93.1) (width 0.16) (layer "B.Cu") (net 7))
 (segment (start 138.4 88.9) (end 137.5 88) (width 0.16) (layer "B.Cu") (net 7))
 (segment (start 145.575 92.9) (end 144.475 94) (width 0.16) (layer "B.Cu") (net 7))
 (segment (start 137.5 88) (end 135.381 88) (width 0.16) (layer "B.Cu") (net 7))
 (via (at 142.4625 92.95) (size 0.6) (drill 0.3) (layers "F.Cu" "B.Cu") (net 5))
 (segment (start 143.45 92.95) (end 144.9 91.5) (width 0.16) (layer "B.Cu") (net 5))
 (segment (start 145.7 91.5) (end 146.619 90.581) (width 0.16) (layer "B.Cu") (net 5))
 (segment (start 142.4625 92.95) (end 143.45 92.95) (width 0.16) (layer "B.Cu") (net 5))
 (segment (start 144.9 91.5) (end 145.7 91.5) (width 0.16) (layer "B.Cu") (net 5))
 (segment (start 146.619 90.581) (end 146.619 88) (width 0.16) (layer "B.Cu") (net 5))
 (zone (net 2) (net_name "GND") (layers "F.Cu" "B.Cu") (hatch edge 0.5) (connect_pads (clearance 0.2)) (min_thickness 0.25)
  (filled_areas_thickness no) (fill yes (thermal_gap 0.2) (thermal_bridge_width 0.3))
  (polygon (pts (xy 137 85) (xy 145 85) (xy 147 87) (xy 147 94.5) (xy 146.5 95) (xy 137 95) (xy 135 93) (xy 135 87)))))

